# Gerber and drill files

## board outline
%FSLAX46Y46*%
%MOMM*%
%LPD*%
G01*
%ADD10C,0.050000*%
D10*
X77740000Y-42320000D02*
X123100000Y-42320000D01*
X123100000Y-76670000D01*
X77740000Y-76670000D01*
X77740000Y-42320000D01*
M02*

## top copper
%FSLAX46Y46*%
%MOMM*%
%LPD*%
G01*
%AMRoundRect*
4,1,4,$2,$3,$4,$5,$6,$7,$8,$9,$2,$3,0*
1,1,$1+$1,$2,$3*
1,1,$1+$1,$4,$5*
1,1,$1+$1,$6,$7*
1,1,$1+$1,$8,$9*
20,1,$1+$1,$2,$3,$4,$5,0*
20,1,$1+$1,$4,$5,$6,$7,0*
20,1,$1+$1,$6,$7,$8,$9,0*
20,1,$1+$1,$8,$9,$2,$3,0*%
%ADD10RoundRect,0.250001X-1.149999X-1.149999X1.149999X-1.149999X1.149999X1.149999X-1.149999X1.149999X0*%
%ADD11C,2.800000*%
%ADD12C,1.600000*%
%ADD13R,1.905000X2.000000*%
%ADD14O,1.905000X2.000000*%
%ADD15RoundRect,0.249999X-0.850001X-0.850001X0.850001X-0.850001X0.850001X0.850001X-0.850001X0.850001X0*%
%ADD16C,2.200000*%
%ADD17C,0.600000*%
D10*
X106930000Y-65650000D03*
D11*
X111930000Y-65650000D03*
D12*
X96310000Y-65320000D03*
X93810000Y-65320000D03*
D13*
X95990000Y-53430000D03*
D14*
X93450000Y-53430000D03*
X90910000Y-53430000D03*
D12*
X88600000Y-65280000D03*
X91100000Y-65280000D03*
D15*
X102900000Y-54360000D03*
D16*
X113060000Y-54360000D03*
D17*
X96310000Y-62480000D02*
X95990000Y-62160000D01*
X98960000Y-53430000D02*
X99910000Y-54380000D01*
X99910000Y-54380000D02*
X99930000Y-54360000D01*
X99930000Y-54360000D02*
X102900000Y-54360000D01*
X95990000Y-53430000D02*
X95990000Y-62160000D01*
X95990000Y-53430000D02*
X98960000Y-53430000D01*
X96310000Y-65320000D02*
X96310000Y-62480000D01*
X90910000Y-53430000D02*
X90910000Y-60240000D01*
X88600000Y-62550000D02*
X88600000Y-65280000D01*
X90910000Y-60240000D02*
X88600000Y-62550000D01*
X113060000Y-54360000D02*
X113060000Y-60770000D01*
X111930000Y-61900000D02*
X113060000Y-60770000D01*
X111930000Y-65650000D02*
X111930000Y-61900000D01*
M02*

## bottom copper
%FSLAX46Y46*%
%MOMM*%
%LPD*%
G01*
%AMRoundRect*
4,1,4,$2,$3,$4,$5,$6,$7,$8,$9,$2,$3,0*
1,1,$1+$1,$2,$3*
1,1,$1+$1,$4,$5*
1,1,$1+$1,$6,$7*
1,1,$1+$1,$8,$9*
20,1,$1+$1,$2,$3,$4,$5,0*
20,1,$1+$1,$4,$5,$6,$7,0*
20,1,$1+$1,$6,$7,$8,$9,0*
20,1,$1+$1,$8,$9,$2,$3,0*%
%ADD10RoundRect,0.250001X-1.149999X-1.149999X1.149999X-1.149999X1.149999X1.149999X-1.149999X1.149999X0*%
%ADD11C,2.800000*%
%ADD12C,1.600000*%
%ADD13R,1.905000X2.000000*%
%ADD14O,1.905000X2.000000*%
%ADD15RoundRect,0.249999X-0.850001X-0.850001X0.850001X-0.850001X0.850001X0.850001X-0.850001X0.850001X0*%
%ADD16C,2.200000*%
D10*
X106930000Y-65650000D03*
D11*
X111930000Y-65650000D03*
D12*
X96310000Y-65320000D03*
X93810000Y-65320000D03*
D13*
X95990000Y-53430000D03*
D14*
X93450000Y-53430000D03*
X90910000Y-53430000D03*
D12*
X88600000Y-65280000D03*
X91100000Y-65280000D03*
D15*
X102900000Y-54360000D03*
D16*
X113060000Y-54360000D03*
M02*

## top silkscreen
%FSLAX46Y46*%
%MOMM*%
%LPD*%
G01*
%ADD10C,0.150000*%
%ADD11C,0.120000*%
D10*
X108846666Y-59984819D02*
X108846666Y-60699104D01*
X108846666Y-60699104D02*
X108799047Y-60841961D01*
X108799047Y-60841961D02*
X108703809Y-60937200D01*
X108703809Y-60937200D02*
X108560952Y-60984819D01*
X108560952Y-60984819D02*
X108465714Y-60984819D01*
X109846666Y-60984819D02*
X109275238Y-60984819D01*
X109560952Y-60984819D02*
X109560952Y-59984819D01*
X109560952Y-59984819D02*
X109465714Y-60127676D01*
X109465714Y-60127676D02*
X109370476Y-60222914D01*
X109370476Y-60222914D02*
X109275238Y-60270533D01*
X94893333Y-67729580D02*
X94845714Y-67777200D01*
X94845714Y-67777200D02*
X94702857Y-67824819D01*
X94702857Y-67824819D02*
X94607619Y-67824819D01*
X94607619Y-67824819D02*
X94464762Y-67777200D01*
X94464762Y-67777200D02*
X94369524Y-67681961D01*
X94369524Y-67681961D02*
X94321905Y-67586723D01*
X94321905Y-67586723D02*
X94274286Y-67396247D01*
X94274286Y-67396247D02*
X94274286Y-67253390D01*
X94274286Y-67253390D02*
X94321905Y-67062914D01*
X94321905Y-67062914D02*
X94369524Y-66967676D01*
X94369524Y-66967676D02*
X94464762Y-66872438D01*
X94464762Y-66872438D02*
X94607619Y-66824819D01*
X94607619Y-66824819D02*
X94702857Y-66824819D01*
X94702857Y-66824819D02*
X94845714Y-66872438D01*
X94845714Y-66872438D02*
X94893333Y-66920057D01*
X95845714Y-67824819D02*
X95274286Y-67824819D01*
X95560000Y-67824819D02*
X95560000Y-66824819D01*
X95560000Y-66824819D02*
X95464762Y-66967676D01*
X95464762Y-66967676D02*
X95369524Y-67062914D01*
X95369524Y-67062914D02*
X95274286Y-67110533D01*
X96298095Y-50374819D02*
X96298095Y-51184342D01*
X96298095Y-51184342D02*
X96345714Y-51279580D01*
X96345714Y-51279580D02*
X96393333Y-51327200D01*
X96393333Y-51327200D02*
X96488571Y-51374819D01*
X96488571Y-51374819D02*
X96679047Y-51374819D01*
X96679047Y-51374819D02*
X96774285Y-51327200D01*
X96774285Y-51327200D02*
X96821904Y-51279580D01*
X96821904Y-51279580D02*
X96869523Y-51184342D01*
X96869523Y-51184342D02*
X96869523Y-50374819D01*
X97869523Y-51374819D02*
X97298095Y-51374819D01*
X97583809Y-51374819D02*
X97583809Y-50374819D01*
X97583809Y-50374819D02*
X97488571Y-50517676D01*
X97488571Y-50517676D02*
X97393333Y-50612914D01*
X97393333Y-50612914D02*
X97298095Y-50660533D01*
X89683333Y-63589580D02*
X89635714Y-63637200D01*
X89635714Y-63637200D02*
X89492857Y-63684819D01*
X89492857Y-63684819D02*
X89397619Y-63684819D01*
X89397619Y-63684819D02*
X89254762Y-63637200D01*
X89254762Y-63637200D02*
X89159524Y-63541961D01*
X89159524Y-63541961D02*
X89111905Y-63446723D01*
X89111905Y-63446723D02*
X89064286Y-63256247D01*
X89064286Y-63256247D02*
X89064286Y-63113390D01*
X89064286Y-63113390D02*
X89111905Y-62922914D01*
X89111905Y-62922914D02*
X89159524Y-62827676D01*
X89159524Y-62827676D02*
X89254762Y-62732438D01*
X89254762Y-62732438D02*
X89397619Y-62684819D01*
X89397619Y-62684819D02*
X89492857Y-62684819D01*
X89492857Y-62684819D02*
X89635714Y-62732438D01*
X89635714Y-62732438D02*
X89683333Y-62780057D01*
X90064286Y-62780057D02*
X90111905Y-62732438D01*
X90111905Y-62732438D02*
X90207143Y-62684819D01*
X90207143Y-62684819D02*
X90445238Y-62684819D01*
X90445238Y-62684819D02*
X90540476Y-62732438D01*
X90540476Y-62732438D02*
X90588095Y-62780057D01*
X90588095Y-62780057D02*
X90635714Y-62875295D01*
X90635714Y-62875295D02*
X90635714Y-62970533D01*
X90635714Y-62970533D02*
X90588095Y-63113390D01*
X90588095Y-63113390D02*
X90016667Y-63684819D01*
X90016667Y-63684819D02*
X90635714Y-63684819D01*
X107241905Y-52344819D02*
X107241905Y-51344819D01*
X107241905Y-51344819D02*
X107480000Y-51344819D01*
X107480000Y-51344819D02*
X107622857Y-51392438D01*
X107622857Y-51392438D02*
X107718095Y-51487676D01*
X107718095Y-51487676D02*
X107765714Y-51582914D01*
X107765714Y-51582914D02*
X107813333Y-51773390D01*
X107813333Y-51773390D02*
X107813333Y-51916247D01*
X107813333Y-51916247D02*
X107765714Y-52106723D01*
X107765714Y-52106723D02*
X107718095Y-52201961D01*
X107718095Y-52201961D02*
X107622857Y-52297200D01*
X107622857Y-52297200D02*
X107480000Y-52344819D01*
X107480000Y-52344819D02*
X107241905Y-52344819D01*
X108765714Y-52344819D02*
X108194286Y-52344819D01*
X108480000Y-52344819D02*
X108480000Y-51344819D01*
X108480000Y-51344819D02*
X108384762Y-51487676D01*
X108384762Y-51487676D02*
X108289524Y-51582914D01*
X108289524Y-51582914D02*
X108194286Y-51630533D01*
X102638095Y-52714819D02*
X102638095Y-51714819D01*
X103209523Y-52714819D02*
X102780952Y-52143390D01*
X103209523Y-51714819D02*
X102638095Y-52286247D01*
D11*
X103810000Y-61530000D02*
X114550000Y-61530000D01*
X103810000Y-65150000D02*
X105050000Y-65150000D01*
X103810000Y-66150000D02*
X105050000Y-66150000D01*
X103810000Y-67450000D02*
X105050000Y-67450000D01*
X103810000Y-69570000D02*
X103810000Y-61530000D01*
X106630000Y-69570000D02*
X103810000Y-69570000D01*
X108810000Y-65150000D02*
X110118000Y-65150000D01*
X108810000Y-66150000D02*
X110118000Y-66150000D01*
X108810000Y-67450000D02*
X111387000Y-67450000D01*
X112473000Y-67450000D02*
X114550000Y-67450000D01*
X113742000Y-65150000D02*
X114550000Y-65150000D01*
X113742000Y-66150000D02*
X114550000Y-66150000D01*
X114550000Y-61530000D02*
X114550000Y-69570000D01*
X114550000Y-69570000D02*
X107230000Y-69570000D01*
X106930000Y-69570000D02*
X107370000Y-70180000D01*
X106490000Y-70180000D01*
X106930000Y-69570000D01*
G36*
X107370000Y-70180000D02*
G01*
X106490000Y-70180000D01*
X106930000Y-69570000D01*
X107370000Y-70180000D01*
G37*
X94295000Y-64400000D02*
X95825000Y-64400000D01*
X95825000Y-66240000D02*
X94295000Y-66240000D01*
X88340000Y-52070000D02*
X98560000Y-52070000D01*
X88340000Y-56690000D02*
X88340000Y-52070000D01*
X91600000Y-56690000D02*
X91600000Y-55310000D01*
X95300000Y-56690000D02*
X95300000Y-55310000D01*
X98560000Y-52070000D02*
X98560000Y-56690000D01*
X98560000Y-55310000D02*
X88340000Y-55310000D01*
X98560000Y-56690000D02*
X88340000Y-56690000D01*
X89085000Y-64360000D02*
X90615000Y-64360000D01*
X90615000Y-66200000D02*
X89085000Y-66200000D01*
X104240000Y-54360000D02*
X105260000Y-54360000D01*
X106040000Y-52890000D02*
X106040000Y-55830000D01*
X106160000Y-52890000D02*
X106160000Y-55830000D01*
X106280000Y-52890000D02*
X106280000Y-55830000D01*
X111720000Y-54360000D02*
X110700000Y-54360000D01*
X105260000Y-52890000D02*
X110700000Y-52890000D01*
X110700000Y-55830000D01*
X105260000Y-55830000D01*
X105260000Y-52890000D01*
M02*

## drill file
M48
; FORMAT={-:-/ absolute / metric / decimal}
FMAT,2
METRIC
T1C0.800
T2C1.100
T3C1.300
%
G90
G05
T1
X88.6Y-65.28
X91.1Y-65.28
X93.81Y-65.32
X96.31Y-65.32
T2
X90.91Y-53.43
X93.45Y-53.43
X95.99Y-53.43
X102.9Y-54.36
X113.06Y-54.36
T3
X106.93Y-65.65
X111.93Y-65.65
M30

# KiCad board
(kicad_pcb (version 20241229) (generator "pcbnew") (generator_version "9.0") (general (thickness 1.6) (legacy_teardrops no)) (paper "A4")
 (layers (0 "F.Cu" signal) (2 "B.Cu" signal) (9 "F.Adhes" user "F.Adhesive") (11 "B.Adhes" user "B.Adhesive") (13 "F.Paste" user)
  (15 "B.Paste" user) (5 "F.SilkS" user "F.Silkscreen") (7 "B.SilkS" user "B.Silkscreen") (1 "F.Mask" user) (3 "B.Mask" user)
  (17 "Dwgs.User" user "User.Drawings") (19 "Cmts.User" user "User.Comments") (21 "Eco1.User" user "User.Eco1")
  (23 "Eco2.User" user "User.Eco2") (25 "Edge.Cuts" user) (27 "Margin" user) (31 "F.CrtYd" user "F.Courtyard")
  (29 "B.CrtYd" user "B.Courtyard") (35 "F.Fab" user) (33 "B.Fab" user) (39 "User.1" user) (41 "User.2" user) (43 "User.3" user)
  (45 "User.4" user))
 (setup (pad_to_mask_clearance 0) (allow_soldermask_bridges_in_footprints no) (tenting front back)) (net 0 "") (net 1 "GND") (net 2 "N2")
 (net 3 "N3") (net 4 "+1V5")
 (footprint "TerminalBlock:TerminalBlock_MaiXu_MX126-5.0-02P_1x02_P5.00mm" (layer "F.Cu") (at 106.93 65.65)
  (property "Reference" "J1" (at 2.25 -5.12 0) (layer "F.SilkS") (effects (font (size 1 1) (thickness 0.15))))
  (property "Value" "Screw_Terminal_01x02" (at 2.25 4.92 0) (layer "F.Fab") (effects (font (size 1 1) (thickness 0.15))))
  (fp_line (start -3.12 -4.12) (end 7.62 -4.12) (stroke (width 0.12) (type solid)) (layer "F.SilkS"))
  (fp_line (start -3.12 -0.5) (end -1.88 -0.5) (stroke (width 0.12) (type solid)) (layer "F.SilkS"))
  (fp_line (start -3.12 0.5) (end -1.88 0.5) (stroke (width 0.12) (type solid)) (layer "F.SilkS"))
  (fp_line (start -3.12 1.8) (end -1.88 1.8) (stroke (width 0.12) (type solid)) (layer "F.SilkS"))
  (fp_line (start -3.12 3.92) (end -3.12 -4.12) (stroke (width 0.12) (type solid)) (layer "F.SilkS"))
  (fp_line (start -0.3 3.92) (end -3.12 3.92) (stroke (width 0.12) (type solid)) (layer "F.SilkS"))
  (fp_line (start 1.88 -0.5) (end 3.188 -0.5) (stroke (width 0.12) (type solid)) (layer "F.SilkS"))
  (fp_line (start 1.88 0.5) (end 3.188 0.5) (stroke (width 0.12) (type solid)) (layer "F.SilkS"))
  (fp_line (start 1.88 1.8) (end 4.457 1.8) (stroke (width 0.12) (type solid)) (layer "F.SilkS"))
  (fp_line (start 5.543 1.8) (end 7.62 1.8) (stroke (width 0.12) (type solid)) (layer "F.SilkS"))
  (fp_line (start 6.812 -0.5) (end 7.62 -0.5) (stroke (width 0.12) (type solid)) (layer "F.SilkS"))
  (fp_line (start 6.812 0.5) (end 7.62 0.5) (stroke (width 0.12) (type solid)) (layer "F.SilkS"))
  (fp_line (start 7.62 -4.12) (end 7.62 3.92) (stroke (width 0.12) (type solid)) (layer "F.SilkS"))
  (fp_line (start 7.62 3.92) (end 0.3 3.92) (stroke (width 0.12) (type solid)) (layer "F.SilkS"))
  (fp_poly (pts (xy 0 3.92) (xy 0.44 4.53) (xy -0.44 4.53)) (stroke (width 0.12) (type solid)) (fill yes) (layer "F.SilkS"))
  (pad "1" thru_hole roundrect (at 0 0) (size 2.8 2.8) (drill 1.3) (layers "*.Cu" "*.Mask") (remove_unused_layers no)
   (roundrect_rratio 0.089286) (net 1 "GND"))
  (pad "2" thru_hole circle (at 5 0) (size 2.8 2.8) (drill 1.3) (layers "*.Cu" "*.Mask") (remove_unused_layers no) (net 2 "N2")))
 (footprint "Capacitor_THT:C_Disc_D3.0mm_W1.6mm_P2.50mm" (layer "F.Cu") (at 96.31 65.32 180)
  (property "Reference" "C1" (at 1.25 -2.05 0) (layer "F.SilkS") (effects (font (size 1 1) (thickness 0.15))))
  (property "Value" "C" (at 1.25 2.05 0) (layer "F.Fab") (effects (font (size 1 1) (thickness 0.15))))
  (fp_line (start 2.015 0.92) (end 0.485 0.92) (stroke (width 0.12) (type solid)) (layer "F.SilkS"))
  (fp_line (start 0.485 -0.92) (end 2.015 -0.92) (stroke (width 0.12) (type solid)) (layer "F.SilkS"))
  (pad "1" thru_hole circle (at 0 0 180) (size 1.6 1.6) (drill 0.8) (layers "*.Cu" "*.Mask") (remove_unused_layers no) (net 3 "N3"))
  (pad "2" thru_hole circle (at 2.5 0 180) (size 1.6 1.6) (drill 0.8) (layers "*.Cu" "*.Mask") (remove_unused_layers no) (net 1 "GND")))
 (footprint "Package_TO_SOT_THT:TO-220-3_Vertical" (layer "F.Cu") (at 95.99 53.43 180)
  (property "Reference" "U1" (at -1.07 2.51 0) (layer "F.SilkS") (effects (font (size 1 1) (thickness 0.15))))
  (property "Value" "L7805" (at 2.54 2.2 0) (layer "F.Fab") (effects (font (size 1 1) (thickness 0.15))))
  (fp_line (start 7.65 1.36) (end -2.57 1.36) (stroke (width 0.12) (type solid)) (layer "F.SilkS"))
  (fp_line (start 7.65 -3.26) (end 7.65 1.36) (stroke (width 0.12) (type solid)) (layer "F.SilkS"))
  (fp_line (start 4.39 -3.26) (end 4.39 -1.88) (stroke (width 0.12) (type solid)) (layer "F.SilkS"))
  (fp_line (start 0.69 -3.26) (end 0.69 -1.88) (stroke (width 0.12) (type solid)) (layer "F.SilkS"))
  (fp_line (start -2.57 1.36) (end -2.57 -3.26) (stroke (width 0.12) (type solid)) (layer "F.SilkS"))
  (fp_line (start -2.57 -1.88) (end 7.65 -1.88) (stroke (width 0.12) (type solid)) (layer "F.SilkS"))
  (fp_line (start -2.57 -3.26) (end 7.65 -3.26) (stroke (width 0.12) (type solid)) (layer "F.SilkS"))
  (pad "1" thru_hole rect (at 0 0 180) (size 1.905 2) (drill 1.1) (layers "*.Cu" "*.Mask") (remove_unused_layers no) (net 3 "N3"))
  (pad "2" thru_hole oval (at 2.54 0 180) (size 1.905 2) (drill 1.1) (layers "*.Cu" "*.Mask") (remove_unused_layers no) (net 1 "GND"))
  (pad "3" thru_hole oval (at 5.08 0 180) (size 1.905 2) (drill 1.1) (layers "*.Cu" "*.Mask") (remove_unused_layers no) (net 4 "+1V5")))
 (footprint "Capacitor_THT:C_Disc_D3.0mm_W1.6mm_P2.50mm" (layer "F.Cu") (at 88.6 65.28)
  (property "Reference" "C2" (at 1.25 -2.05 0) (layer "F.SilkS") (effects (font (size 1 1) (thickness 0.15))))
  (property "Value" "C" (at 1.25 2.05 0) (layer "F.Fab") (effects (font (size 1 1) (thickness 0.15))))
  (fp_line (start 0.485 -0.92) (end 2.015 -0.92) (stroke (width 0.12) (type solid)) (layer "F.SilkS"))
  (fp_line (start 2.015 0.92) (end 0.485 0.92) (stroke (width 0.12) (type solid)) (layer "F.SilkS"))
  (pad "1" thru_hole circle (at 0 0) (size 1.6 1.6) (drill 0.8) (layers "*.Cu" "*.Mask") (remove_unused_layers no) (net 4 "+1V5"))
  (pad "2" thru_hole circle (at 2.5 0) (size 1.6 1.6) (drill 0.8) (layers "*.Cu" "*.Mask") (remove_unused_layers no) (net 1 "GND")))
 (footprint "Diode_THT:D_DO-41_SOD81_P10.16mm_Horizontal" (layer "F.Cu") (at 102.9 54.36)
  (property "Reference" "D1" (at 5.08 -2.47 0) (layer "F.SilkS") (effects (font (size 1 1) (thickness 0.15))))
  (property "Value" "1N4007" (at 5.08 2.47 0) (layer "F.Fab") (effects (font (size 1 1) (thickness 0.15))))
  (fp_line (start 1.34 0) (end 2.36 0) (stroke (width 0.12) (type solid)) (layer "F.SilkS"))
  (fp_line (start 3.14 -1.47) (end 3.14 1.47) (stroke (width 0.12) (type solid)) (layer "F.SilkS"))
  (fp_line (start 3.26 -1.47) (end 3.26 1.47) (stroke (width 0.12) (type solid)) (layer "F.SilkS"))
  (fp_line (start 3.38 -1.47) (end 3.38 1.47) (stroke (width 0.12) (type solid)) (layer "F.SilkS"))
  (fp_line (start 8.82 0) (end 7.8 0) (stroke (width 0.12) (type solid)) (layer "F.SilkS"))
  (fp_rect (start 2.36 -1.47) (end 7.8 1.47) (stroke (width 0.12) (type solid)) (fill no) (layer "F.SilkS"))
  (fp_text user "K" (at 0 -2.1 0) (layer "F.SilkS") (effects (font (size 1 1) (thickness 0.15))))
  (pad "1" thru_hole roundrect (at 0 0) (size 2.2 2.2) (drill 1.1) (layers "*.Cu" "*.Mask") (remove_unused_layers no)
   (roundrect_rratio 0.113636) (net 3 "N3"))
  (pad "2" thru_hole circle (at 10.16 0) (size 2.2 2.2) (drill 1.1) (layers "*.Cu" "*.Mask") (remove_unused_layers no) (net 2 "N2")))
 (gr_rect (start 77.74 42.32) (end 123.1 76.67) (stroke (width 0.05) (type default)) (fill no) (layer "Edge.Cuts"))
 (segment (start 96.31 62.48) (end 95.99 62.16) (width 0.6) (layer "F.Cu") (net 3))
 (segment (start 98.96 53.43) (end 99.91 54.38) (width 0.6) (layer "F.Cu") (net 3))
 (segment (start 99.91 54.38) (end 99.93 54.36) (width 0.6) (layer "F.Cu") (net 3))
 (segment (start 99.93 54.36) (end 102.9 54.36) (width 0.6) (layer "F.Cu") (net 3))
 (segment (start 95.99 53.43) (end 95.99 62.16) (width 0.6) (layer "F.Cu") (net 3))
 (segment (start 95.99 53.43) (end 98.96 53.43) (width 0.6) (layer "F.Cu") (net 3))
 (segment (start 96.31 65.32) (end 96.31 62.48) (width 0.6) (layer "F.Cu") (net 3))
 (segment (start 90.91 53.43) (end 90.91 60.24) (width 0.6) (layer "F.Cu") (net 4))
 (segment (start 88.6 62.55) (end 88.6 65.28) (width 0.6) (layer "F.Cu") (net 4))
 (segment (start 90.91 60.24) (end 88.6 62.55) (width 0.6) (layer "F.Cu") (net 4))
 (segment (start 113.06 54.36) (end 113.06 60.77) (width 0.6) (layer "F.Cu") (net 2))
 (segment (start 111.93 61.9) (end 113.06 60.77) (width 0.6) (layer "F.Cu") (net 2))
 (segment (start 111.93 65.65) (end 111.93 61.9) (width 0.6) (layer "F.Cu") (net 2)))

